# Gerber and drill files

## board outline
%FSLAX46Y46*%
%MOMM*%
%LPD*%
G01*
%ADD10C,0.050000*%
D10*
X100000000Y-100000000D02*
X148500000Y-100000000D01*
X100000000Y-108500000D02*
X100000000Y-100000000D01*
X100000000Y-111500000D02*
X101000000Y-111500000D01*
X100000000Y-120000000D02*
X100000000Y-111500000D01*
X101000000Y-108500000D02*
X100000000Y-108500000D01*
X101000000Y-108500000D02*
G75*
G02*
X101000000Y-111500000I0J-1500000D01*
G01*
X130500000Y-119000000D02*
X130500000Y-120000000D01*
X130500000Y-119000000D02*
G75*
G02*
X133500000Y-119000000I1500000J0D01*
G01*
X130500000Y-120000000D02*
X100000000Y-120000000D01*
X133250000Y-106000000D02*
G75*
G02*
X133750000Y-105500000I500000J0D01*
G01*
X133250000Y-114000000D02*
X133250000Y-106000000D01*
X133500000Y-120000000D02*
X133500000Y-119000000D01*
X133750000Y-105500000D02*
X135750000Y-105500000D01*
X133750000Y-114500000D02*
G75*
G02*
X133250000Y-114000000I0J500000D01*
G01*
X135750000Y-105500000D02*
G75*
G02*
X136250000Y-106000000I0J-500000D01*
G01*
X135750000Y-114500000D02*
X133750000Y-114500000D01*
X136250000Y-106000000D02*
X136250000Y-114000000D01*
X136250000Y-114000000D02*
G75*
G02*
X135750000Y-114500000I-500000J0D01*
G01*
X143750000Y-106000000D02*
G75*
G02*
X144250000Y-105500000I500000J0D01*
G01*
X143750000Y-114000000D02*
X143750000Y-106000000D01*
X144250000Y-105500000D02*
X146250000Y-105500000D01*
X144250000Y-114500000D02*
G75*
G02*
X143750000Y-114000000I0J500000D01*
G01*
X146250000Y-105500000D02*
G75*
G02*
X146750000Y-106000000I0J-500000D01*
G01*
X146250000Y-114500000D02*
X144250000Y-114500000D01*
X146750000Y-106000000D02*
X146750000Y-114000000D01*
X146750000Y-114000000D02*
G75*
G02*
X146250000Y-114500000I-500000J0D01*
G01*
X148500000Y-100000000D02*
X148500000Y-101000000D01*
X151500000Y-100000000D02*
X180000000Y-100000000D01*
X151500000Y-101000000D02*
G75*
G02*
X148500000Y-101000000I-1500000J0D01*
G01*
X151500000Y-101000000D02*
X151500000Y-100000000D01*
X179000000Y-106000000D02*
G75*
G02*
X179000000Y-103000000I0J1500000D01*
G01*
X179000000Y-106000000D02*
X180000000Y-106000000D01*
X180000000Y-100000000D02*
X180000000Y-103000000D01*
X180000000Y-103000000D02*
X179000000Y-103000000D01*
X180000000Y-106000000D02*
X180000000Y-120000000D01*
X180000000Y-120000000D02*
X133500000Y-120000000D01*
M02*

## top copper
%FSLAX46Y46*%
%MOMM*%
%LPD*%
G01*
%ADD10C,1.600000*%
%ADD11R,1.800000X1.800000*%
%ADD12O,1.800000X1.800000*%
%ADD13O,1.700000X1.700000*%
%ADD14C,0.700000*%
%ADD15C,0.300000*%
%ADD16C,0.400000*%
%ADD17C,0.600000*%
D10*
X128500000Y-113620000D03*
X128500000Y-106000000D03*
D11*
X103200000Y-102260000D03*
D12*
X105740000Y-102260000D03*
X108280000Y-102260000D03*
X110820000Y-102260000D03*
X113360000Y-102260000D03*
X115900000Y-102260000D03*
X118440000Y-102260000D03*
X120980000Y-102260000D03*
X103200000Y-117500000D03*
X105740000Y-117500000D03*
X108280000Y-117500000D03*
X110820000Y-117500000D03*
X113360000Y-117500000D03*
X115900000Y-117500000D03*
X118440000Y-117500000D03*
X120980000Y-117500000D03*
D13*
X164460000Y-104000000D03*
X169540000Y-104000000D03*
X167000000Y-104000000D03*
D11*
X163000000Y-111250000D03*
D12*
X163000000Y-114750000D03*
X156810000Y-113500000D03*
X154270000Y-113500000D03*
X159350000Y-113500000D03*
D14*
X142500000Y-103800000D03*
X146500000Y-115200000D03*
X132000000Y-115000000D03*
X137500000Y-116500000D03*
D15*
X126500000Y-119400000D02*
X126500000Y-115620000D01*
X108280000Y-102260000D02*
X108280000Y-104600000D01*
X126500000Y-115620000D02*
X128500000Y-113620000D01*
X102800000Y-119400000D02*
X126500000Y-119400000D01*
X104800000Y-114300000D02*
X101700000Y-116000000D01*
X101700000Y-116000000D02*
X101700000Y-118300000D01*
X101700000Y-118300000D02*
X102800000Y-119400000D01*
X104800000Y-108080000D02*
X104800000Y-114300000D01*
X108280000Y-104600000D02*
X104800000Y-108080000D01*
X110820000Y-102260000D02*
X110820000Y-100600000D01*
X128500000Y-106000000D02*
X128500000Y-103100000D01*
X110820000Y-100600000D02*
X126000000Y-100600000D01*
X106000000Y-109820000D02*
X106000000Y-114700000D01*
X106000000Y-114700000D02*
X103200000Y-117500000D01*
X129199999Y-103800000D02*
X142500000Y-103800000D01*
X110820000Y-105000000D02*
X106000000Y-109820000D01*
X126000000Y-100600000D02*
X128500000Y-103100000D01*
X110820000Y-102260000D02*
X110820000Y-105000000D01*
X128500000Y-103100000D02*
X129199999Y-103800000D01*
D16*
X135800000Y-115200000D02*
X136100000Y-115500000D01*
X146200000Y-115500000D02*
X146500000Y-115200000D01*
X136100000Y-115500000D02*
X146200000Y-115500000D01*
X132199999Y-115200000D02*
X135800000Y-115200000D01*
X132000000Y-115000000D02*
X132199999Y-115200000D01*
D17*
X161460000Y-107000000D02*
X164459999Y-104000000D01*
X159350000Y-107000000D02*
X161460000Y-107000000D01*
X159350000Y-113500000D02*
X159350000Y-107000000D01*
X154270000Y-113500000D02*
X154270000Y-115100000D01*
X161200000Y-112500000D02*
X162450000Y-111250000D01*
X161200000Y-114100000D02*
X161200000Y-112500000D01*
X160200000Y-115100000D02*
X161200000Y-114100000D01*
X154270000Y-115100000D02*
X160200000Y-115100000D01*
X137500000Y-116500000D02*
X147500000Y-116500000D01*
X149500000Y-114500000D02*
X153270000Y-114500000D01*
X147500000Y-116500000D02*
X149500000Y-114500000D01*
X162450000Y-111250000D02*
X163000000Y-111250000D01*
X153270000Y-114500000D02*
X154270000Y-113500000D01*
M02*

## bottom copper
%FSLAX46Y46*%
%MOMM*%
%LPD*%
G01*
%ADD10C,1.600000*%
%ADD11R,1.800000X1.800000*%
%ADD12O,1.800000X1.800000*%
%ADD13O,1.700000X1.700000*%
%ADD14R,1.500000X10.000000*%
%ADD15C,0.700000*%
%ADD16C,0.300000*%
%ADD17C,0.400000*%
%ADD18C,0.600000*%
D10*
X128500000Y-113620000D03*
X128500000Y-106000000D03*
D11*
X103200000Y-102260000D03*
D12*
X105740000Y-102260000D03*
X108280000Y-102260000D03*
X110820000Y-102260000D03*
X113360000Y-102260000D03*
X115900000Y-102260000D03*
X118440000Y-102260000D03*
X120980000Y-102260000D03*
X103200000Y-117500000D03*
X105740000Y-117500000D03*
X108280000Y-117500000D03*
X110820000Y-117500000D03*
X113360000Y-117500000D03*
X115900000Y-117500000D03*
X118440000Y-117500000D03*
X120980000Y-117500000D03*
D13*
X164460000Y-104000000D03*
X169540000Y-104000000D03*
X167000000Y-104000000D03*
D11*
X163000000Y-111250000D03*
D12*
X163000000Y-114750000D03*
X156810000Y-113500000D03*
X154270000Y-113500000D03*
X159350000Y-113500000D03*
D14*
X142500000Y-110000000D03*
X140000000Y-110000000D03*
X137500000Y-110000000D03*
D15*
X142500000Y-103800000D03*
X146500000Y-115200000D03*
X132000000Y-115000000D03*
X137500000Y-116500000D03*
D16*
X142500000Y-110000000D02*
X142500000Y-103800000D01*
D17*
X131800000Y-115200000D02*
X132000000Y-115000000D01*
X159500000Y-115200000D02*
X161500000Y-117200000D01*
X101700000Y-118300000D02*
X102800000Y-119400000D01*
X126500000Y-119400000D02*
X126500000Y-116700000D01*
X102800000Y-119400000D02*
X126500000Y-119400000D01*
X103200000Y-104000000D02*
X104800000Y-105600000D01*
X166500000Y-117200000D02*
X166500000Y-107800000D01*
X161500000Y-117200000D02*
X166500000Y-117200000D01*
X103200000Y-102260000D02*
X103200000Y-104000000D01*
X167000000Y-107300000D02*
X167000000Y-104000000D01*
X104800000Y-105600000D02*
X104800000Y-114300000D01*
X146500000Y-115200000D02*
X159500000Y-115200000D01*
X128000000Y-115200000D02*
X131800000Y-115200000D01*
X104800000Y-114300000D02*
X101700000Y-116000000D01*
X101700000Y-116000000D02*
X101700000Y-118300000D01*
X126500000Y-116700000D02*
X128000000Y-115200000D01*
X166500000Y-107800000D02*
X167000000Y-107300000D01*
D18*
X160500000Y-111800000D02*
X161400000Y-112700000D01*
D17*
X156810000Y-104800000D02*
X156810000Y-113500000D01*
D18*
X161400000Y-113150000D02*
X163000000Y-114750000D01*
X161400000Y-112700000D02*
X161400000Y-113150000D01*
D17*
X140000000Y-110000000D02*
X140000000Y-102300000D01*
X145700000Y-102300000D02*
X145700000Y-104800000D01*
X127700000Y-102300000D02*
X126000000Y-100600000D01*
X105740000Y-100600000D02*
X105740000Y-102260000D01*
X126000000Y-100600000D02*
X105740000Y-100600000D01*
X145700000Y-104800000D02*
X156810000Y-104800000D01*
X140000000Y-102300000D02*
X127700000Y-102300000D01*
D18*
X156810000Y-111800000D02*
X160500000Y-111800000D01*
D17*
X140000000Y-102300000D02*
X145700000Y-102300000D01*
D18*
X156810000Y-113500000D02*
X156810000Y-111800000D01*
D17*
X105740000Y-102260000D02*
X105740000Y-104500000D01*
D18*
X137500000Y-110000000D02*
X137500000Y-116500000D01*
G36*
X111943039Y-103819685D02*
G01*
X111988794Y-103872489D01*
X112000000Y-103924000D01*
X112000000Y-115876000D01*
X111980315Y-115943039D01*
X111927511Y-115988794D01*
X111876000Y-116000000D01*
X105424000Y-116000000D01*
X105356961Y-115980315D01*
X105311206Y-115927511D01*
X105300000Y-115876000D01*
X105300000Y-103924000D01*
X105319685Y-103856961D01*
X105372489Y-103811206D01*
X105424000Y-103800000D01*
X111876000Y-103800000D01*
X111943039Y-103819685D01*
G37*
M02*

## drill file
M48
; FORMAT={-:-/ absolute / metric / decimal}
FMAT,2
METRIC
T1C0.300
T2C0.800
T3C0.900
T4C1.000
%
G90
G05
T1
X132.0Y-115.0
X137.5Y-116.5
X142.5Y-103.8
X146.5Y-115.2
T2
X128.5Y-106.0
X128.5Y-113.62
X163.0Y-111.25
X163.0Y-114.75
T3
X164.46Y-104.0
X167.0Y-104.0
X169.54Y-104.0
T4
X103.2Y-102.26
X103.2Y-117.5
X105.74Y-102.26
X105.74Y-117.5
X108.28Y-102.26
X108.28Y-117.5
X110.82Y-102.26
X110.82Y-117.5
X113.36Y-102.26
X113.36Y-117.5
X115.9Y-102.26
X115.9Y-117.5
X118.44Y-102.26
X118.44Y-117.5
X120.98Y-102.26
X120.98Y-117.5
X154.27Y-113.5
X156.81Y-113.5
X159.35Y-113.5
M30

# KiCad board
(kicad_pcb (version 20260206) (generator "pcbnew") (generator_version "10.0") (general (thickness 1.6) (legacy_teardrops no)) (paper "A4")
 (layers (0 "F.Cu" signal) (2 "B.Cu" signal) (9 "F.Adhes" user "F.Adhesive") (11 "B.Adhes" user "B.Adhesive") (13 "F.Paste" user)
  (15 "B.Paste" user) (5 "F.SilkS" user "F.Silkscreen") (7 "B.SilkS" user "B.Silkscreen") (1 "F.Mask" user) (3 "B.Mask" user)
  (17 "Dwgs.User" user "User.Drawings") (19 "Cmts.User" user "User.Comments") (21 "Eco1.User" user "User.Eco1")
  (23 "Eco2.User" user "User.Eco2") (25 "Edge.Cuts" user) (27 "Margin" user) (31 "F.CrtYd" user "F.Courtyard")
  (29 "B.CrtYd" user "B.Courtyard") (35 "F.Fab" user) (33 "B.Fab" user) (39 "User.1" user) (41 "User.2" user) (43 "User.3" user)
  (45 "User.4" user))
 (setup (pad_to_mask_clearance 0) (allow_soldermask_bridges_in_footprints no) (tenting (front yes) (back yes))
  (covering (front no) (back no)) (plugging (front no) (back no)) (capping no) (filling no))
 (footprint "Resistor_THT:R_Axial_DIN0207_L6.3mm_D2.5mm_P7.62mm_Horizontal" (layer "F.Cu") (at 128.5 113.62 90)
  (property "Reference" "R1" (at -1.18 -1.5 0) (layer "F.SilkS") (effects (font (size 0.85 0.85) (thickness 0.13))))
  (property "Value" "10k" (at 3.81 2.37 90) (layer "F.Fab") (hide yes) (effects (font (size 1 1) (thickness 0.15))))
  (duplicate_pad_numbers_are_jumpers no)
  (pad "1" thru_hole circle (at 0 0 90) (size 1.6 1.6) (drill 0.8) (layers "*.Cu" "*.Mask") (remove_unused_layers no) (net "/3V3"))
  (pad "2" thru_hole circle (at 7.62 0 90) (size 1.6 1.6) (drill 0.8) (layers "*.Cu" "*.Mask") (remove_unused_layers no) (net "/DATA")))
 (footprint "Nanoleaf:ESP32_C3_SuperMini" (layer "F.Cu") (at 103.2 117.5 90)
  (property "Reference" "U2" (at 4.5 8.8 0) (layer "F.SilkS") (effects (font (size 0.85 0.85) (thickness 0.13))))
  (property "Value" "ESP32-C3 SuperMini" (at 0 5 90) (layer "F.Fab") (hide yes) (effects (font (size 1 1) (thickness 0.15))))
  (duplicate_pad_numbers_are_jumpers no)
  (pad "1" thru_hole rect (at 15.24 0 90) (size 1.8 1.8) (drill 1) (layers "*.Cu" "*.Mask") (remove_unused_layers no) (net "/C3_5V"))
  (pad "2" thru_hole oval (at 15.24 2.54 90) (size 1.8 1.8) (drill 1) (layers "*.Cu" "*.Mask") (remove_unused_layers no) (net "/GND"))
  (pad "3" thru_hole oval (at 15.24 5.08 90) (size 1.8 1.8) (drill 1) (layers "*.Cu" "*.Mask") (remove_unused_layers no) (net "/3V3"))
  (pad "4" thru_hole oval (at 15.24 7.62 90) (size 1.8 1.8) (drill 1) (layers "*.Cu" "*.Mask") (remove_unused_layers no) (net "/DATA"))
  (pad "5" thru_hole oval (at 15.24 10.16 90) (size 1.8 1.8) (drill 1) (layers "*.Cu" "*.Mask") (remove_unused_layers no)
   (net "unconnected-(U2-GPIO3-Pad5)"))
  (pad "6" thru_hole oval (at 15.24 12.7 90) (size 1.8 1.8) (drill 1) (layers "*.Cu" "*.Mask") (remove_unused_layers no)
   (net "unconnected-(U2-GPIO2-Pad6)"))
  (pad "7" thru_hole oval (at 15.24 15.24 90) (size 1.8 1.8) (drill 1) (layers "*.Cu" "*.Mask") (remove_unused_layers no)
   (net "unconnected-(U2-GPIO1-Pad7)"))
  (pad "8" thru_hole oval (at 15.24 17.78 90) (size 1.8 1.8) (drill 1) (layers "*.Cu" "*.Mask") (remove_unused_layers no)
   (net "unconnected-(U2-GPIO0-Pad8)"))
  (pad "9" thru_hole oval (at 0 0 90) (size 1.8 1.8) (drill 1) (layers "*.Cu" "*.Mask") (remove_unused_layers no) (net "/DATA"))
  (pad "10" thru_hole oval (at 0 2.54 90) (size 1.8 1.8) (drill 1) (layers "*.Cu" "*.Mask") (remove_unused_layers no)
   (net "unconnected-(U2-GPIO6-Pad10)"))
  (pad "11" thru_hole oval (at 0 5.08 90) (size 1.8 1.8) (drill 1) (layers "*.Cu" "*.Mask") (remove_unused_layers no)
   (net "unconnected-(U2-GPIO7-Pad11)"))
  (pad "12" thru_hole oval (at 0 7.62 90) (size 1.8 1.8) (drill 1) (layers "*.Cu" "*.Mask") (remove_unused_layers no)
   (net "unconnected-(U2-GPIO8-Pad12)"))
  (pad "13" thru_hole oval (at 0 10.16 90) (size 1.8 1.8) (drill 1) (layers "*.Cu" "*.Mask") (remove_unused_layers no)
   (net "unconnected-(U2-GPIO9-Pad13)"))
  (pad "14" thru_hole oval (at 0 12.7 90) (size 1.8 1.8) (drill 1) (layers "*.Cu" "*.Mask") (remove_unused_layers no)
   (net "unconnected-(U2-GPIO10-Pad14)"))
  (pad "15" thru_hole oval (at 0 15.24 90) (size 1.8 1.8) (drill 1) (layers "*.Cu" "*.Mask") (remove_unused_layers no)
   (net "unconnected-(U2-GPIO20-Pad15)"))
  (pad "16" thru_hole oval (at 0 17.78 90) (size 1.8 1.8) (drill 1) (layers "*.Cu" "*.Mask") (remove_unused_layers no)
   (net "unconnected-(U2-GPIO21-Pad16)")))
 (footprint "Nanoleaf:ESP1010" (layer "F.Cu") (at 167 104)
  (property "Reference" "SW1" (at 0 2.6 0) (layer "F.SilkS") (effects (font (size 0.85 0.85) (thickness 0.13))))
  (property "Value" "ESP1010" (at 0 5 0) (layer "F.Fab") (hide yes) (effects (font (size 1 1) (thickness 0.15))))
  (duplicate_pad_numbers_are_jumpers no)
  (pad "1" thru_hole oval (at -2.54 0) (size 1.7 1.7) (drill 0.9) (layers "*.Cu" "*.Mask") (remove_unused_layers no) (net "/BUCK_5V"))
  (pad "2" thru_hole oval (at 2.54 0) (size 1.7 1.7) (drill 0.9) (layers "*.Cu" "*.Mask") (remove_unused_layers no)
   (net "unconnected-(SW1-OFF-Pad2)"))
  (pad "C" thru_hole oval (at 0 0) (size 1.7 1.7) (drill 0.9) (layers "*.Cu" "*.Mask") (remove_unused_layers no) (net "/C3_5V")))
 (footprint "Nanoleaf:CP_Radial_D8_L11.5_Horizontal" (layer "F.Cu") (at 163 111.25)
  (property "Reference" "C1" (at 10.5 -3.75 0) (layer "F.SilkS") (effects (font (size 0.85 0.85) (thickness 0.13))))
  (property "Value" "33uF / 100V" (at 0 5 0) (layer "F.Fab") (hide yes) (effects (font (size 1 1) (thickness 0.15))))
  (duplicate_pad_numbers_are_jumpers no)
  (pad "1" thru_hole rect (at 0 0) (size 1.8 1.8) (drill 0.8) (layers "*.Cu" "*.Mask") (remove_unused_layers no) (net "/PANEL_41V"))
  (pad "2" thru_hole oval (at 0 3.5) (size 1.8 1.8) (drill 0.8) (layers "*.Cu" "*.Mask") (remove_unused_layers no) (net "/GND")))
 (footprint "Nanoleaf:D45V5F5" (layer "F.Cu") (at 154.27 113.5)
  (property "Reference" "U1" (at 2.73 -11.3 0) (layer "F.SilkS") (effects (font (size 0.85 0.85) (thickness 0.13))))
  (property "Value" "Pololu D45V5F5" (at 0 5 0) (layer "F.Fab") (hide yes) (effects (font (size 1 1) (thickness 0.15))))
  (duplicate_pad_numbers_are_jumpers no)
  (pad "GND" thru_hole oval (at 2.54 0) (size 1.8 1.8) (drill 1) (layers "*.Cu" "*.Mask") (remove_unused_layers no) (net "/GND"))
  (pad "VIN" thru_hole oval (at 0 0) (size 1.8 1.8) (drill 1) (layers "*.Cu" "*.Mask") (remove_unused_layers no) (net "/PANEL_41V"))
  (pad "VOUT" thru_hole oval (at 5.08 0) (size 1.8 1.8) (drill 1) (layers "*.Cu" "*.Mask") (remove_unused_layers no) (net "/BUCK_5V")))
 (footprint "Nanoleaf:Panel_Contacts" (layer "B.Cu") (at 140 110 180)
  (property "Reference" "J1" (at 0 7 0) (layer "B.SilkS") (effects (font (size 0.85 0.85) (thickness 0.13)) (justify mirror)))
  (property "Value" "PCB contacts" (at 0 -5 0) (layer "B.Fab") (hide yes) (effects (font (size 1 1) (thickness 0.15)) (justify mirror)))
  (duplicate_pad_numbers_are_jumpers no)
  (pad "1" smd rect (at -2.5 0 180) (size 1.5 10) (layers "B.Cu" "B.Mask") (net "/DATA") (solder_mask_margin 0) (clearance 0.4))
  (pad "2" smd rect (at 0 0 180) (size 1.5 10) (layers "B.Cu" "B.Mask") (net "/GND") (solder_mask_margin 0) (clearance 0.4))
  (pad "3" smd rect (at 2.5 0 180) (size 1.5 10) (layers "B.Cu" "B.Mask") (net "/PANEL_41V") (solder_mask_margin 0) (clearance 0.4)))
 (gr_line (start 100 100) (end 148.5 100) (stroke (width 0.05) (type default)) (layer "Edge.Cuts"))
 (gr_line (start 100 108.5) (end 100 100) (stroke (width 0.05) (type default)) (layer "Edge.Cuts"))
 (gr_line (start 100 111.5) (end 101 111.5) (stroke (width 0.05) (type default)) (layer "Edge.Cuts"))
 (gr_line (start 100 120) (end 100 111.5) (stroke (width 0.05) (type default)) (layer "Edge.Cuts"))
 (gr_line (start 101 108.5) (end 100 108.5) (stroke (width 0.05) (type default)) (layer "Edge.Cuts"))
 (gr_arc (start 101 108.5) (mid 102.5 110) (end 101 111.5) (stroke (width 0.05) (type default)) (layer "Edge.Cuts"))
 (gr_line (start 130.5 119) (end 130.5 120) (stroke (width 0.05) (type default)) (layer "Edge.Cuts"))
 (gr_arc (start 130.5 119) (mid 132 117.5) (end 133.5 119) (stroke (width 0.05) (type default)) (layer "Edge.Cuts"))
 (gr_line (start 130.5 120) (end 100 120) (stroke (width 0.05) (type default)) (layer "Edge.Cuts"))
 (gr_arc (start 133.25 106) (mid 133.396446 105.646446) (end 133.75 105.5) (stroke (width 0.05) (type default)) (layer "Edge.Cuts"))
 (gr_line (start 133.25 114) (end 133.25 106) (stroke (width 0.05) (type default)) (layer "Edge.Cuts"))
 (gr_line (start 133.5 120) (end 133.5 119) (stroke (width 0.05) (type default)) (layer "Edge.Cuts"))
 (gr_line (start 133.75 105.5) (end 135.75 105.5) (stroke (width 0.05) (type default)) (layer "Edge.Cuts"))
 (gr_arc (start 133.75 114.5) (mid 133.396446 114.353553) (end 133.25 114) (stroke (width 0.05) (type default)) (layer "Edge.Cuts"))
 (gr_arc (start 135.75 105.5) (mid 136.103553 105.646446) (end 136.25 106) (stroke (width 0.05) (type default)) (layer "Edge.Cuts"))
 (gr_line (start 135.75 114.5) (end 133.75 114.5) (stroke (width 0.05) (type default)) (layer "Edge.Cuts"))
 (gr_line (start 136.25 106) (end 136.25 114) (stroke (width 0.05) (type default)) (layer "Edge.Cuts"))
 (gr_arc (start 136.25 114) (mid 136.103553 114.353553) (end 135.75 114.5) (stroke (width 0.05) (type default)) (layer "Edge.Cuts"))
 (gr_arc (start 143.75 106) (mid 143.896446 105.646446) (end 144.25 105.5) (stroke (width 0.05) (type default)) (layer "Edge.Cuts"))
 (gr_line (start 143.75 114) (end 143.75 106) (stroke (width 0.05) (type default)) (layer "Edge.Cuts"))
 (gr_line (start 144.25 105.5) (end 146.25 105.5) (stroke (width 0.05) (type default)) (layer "Edge.Cuts"))
 (gr_arc (start 144.25 114.5) (mid 143.896446 114.353553) (end 143.75 114) (stroke (width 0.05) (type default)) (layer "Edge.Cuts"))
 (gr_arc (start 146.25 105.5) (mid 146.603553 105.646446) (end 146.75 106) (stroke (width 0.05) (type default)) (layer "Edge.Cuts"))
 (gr_line (start 146.25 114.5) (end 144.25 114.5) (stroke (width 0.05) (type default)) (layer "Edge.Cuts"))
 (gr_line (start 146.75 106) (end 146.75 114) (stroke (width 0.05) (type default)) (layer "Edge.Cuts"))
 (gr_arc (start 146.75 114) (mid 146.603553 114.353553) (end 146.25 114.5) (stroke (width 0.05) (type default)) (layer "Edge.Cuts"))
 (gr_line (start 148.5 100) (end 148.5 101) (stroke (width 0.05) (type default)) (layer "Edge.Cuts"))
 (gr_line (start 151.5 100) (end 180 100) (stroke (width 0.05) (type default)) (layer "Edge.Cuts"))
 (gr_arc (start 151.5 101) (mid 150 102.5) (end 148.5 101) (stroke (width 0.05) (type default)) (layer "Edge.Cuts"))
 (gr_line (start 151.5 101) (end 151.5 100) (stroke (width 0.05) (type default)) (layer "Edge.Cuts"))
 (gr_arc (start 179 106) (mid 177.5 104.5) (end 179 103) (stroke (width 0.05) (type default)) (layer "Edge.Cuts"))
 (gr_line (start 179 106) (end 180 106) (stroke (width 0.05) (type default)) (layer "Edge.Cuts"))
 (gr_line (start 180 100) (end 180 103) (stroke (width 0.05) (type default)) (layer "Edge.Cuts"))
 (gr_line (start 180 103) (end 179 103) (stroke (width 0.05) (type default)) (layer "Edge.Cuts"))
 (gr_line (start 180 106) (end 180 120) (stroke (width 0.05) (type default)) (layer "Edge.Cuts"))
 (gr_line (start 180 120) (end 133.5 120) (stroke (width 0.05) (type default)) (layer "Edge.Cuts"))
 (segment (start 126.5 119.4) (end 126.5 115.62) (width 0.3) (layer "F.Cu") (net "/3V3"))
 (segment (start 108.28 102.26) (end 108.28 104.6) (width 0.3) (layer "F.Cu") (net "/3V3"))
 (segment (start 126.5 115.62) (end 128.5 113.62) (width 0.3) (layer "F.Cu") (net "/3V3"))
 (segment (start 102.8 119.4) (end 126.5 119.4) (width 0.3) (layer "F.Cu") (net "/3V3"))
 (segment (start 104.8 114.3) (end 101.7 116) (width 0.3) (layer "F.Cu") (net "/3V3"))
 (segment (start 101.7 116) (end 101.7 118.3) (width 0.3) (layer "F.Cu") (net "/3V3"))
 (segment (start 101.7 118.3) (end 102.8 119.4) (width 0.3) (layer "F.Cu") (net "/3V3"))
 (segment (start 104.8 108.08) (end 104.8 114.3) (width 0.3) (layer "F.Cu") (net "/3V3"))
 (segment (start 108.28 104.6) (end 104.8 108.08) (width 0.3) (layer "F.Cu") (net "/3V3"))
 (segment (start 110.82 102.26) (end 110.82 100.6) (width 0.3) (layer "F.Cu") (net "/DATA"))
 (segment (start 128.5 106) (end 128.5 103.1) (width 0.3) (layer "F.Cu") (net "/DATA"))
 (segment (start 110.82 100.6) (end 126 100.6) (width 0.3) (layer "F.Cu") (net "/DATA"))
 (segment (start 106 109.82) (end 106 114.7) (width 0.3) (layer "F.Cu") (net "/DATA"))
 (segment (start 106 114.7) (end 103.2 117.5) (width 0.3) (layer "F.Cu") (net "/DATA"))
 (segment (start 129.199999 103.8) (end 142.5 103.8) (width 0.3) (layer "F.Cu") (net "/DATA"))
 (segment (start 110.82 105) (end 106 109.82) (width 0.3) (layer "F.Cu") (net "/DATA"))
 (segment (start 126 100.6) (end 128.5 103.1) (width 0.3) (layer "F.Cu") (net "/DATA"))
 (segment (start 110.82 102.26) (end 110.82 105) (width 0.3) (layer "F.Cu") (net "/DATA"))
 (segment (start 128.5 103.1) (end 129.199999 103.8) (width 0.3) (layer "F.Cu") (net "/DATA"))
 (via (at 142.5 103.8) (size 0.7) (drill 0.3) (layers "F.Cu" "B.Cu") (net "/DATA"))
 (segment (start 142.5 110) (end 142.5 103.8) (width 0.3) (layer "B.Cu") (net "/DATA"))
 (segment (start 135.8 115.2) (end 136.1 115.5) (width 0.4) (layer "F.Cu") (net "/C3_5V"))
 (segment (start 146.2 115.5) (end 146.5 115.2) (width 0.4) (layer "F.Cu") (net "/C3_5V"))
 (segment (start 136.1 115.5) (end 146.2 115.5) (width 0.4) (layer "F.Cu") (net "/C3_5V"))
 (segment (start 132.199999 115.2) (end 135.8 115.2) (width 0.4) (layer "F.Cu") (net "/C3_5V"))
 (segment (start 132 115) (end 132.199999 115.2) (width 0.4) (layer "F.Cu") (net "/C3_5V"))
 (via (at 146.5 115.2) (size 0.7) (drill 0.3) (layers "F.Cu" "B.Cu") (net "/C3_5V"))
 (via (at 132 115) (size 0.7) (drill 0.3) (layers "F.Cu" "B.Cu") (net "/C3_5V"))
 (segment (start 131.8 115.2) (end 132 115) (width 0.4) (layer "B.Cu") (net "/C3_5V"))
 (segment (start 159.5 115.2) (end 161.5 117.2) (width 0.4) (layer "B.Cu") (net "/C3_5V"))
 (segment (start 101.7 118.3) (end 102.8 119.4) (width 0.4) (layer "B.Cu") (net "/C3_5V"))
 (segment (start 126.5 119.4) (end 126.5 116.7) (width 0.4) (layer "B.Cu") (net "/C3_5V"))
 (segment (start 102.8 119.4) (end 126.5 119.4) (width 0.4) (layer "B.Cu") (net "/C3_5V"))
 (segment (start 103.2 104) (end 104.8 105.6) (width 0.4) (layer "B.Cu") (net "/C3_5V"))
 (segment (start 166.5 117.2) (end 166.5 107.8) (width 0.4) (layer "B.Cu") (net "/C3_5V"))
 (segment (start 161.5 117.2) (end 166.5 117.2) (width 0.4) (layer "B.Cu") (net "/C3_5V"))
 (segment (start 103.2 102.26) (end 103.2 104) (width 0.4) (layer "B.Cu") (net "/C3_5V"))
 (segment (start 167 107.3) (end 167 104) (width 0.4) (layer "B.Cu") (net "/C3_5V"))
 (segment (start 104.8 105.6) (end 104.8 114.3) (width 0.4) (layer "B.Cu") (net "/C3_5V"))
 (segment (start 146.5 115.2) (end 159.5 115.2) (width 0.4) (layer "B.Cu") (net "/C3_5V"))
 (segment (start 128 115.2) (end 131.8 115.2) (width 0.4) (layer "B.Cu") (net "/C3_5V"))
 (segment (start 104.8 114.3) (end 101.7 116) (width 0.4) (layer "B.Cu") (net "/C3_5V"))
 (segment (start 101.7 116) (end 101.7 118.3) (width 0.4) (layer "B.Cu") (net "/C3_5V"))
 (segment (start 126.5 116.7) (end 128 115.2) (width 0.4) (layer "B.Cu") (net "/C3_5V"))
 (segment (start 166.5 107.8) (end 167 107.3) (width 0.4) (layer "B.Cu") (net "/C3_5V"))
 (segment (start 160.5 111.8) (end 161.4 112.7) (width 0.6) (layer "B.Cu") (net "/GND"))
 (segment (start 156.81 104.8) (end 156.81 113.5) (width 0.4) (layer "B.Cu") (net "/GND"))
 (segment (start 161.4 113.15) (end 163 114.75) (width 0.6) (layer "B.Cu") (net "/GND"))
 (segment (start 161.4 112.7) (end 161.4 113.15) (width 0.6) (layer "B.Cu") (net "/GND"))
 (segment (start 140 110) (end 140 102.3) (width 0.4) (layer "B.Cu") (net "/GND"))
 (segment (start 145.7 102.3) (end 145.7 104.8) (width 0.4) (layer "B.Cu") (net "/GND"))
 (segment (start 127.7 102.3) (end 126 100.6) (width 0.4) (layer "B.Cu") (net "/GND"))
 (segment (start 105.74 100.6) (end 105.74 102.26) (width 0.4) (layer "B.Cu") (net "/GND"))
 (segment (start 126 100.6) (end 105.74 100.6) (width 0.4) (layer "B.Cu") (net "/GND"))
 (segment (start 145.7 104.8) (end 156.81 104.8) (width 0.4) (layer "B.Cu") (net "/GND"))
 (segment (start 140 102.3) (end 127.7 102.3) (width 0.4) (layer "B.Cu") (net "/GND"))
 (segment (start 156.81 111.8) (end 160.5 111.8) (width 0.6) (layer "B.Cu") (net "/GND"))
 (segment (start 140 102.3) (end 145.7 102.3) (width 0.4) (layer "B.Cu") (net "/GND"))
 (segment (start 156.81 113.5) (end 156.81 111.8) (width 0.6) (layer "B.Cu") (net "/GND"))
 (segment (start 105.74 102.26) (end 105.74 104.5) (width 0.4) (layer "B.Cu") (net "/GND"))
 (segment (start 161.46 107) (end 164.459999 104) (width 0.6) (layer "F.Cu") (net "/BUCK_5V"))
 (segment (start 159.35 107) (end 161.46 107) (width 0.6) (layer "F.Cu") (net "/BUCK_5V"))
 (segment (start 159.35 113.5) (end 159.35 107) (width 0.6) (layer "F.Cu") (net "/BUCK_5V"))
 (segment (start 154.27 113.5) (end 154.27 115.1) (width 0.6) (layer "F.Cu") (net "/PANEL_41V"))
 (segment (start 161.2 112.5) (end 162.45 111.25) (width 0.6) (layer "F.Cu") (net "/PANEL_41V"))
 (segment (start 161.2 114.1) (end 161.2 112.5) (width 0.6) (layer "F.Cu") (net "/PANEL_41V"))
 (segment (start 160.2 115.1) (end 161.2 114.1) (width 0.6) (layer "F.Cu") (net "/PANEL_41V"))
 (segment (start 154.27 115.1) (end 160.2 115.1) (width 0.6) (layer "F.Cu") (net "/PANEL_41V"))
 (segment (start 137.5 116.5) (end 147.5 116.5) (width 0.6) (layer "F.Cu") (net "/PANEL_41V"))
 (segment (start 149.5 114.5) (end 153.27 114.5) (width 0.6) (layer "F.Cu") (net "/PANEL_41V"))
 (segment (start 147.5 116.5) (end 149.5 114.5) (width 0.6) (layer "F.Cu") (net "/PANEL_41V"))
 (segment (start 162.45 111.25) (end 163 111.25) (width 0.6) (layer "F.Cu") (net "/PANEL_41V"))
 (segment (start 153.27 114.5) (end 154.27 113.5) (width 0.6) (layer "F.Cu") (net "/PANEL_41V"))
 (via (at 137.5 116.5) (size 0.7) (drill 0.3) (layers "F.Cu" "B.Cu") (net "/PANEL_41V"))
 (segment (start 137.5 110) (end 137.5 116.5) (width 0.6) (layer "B.Cu") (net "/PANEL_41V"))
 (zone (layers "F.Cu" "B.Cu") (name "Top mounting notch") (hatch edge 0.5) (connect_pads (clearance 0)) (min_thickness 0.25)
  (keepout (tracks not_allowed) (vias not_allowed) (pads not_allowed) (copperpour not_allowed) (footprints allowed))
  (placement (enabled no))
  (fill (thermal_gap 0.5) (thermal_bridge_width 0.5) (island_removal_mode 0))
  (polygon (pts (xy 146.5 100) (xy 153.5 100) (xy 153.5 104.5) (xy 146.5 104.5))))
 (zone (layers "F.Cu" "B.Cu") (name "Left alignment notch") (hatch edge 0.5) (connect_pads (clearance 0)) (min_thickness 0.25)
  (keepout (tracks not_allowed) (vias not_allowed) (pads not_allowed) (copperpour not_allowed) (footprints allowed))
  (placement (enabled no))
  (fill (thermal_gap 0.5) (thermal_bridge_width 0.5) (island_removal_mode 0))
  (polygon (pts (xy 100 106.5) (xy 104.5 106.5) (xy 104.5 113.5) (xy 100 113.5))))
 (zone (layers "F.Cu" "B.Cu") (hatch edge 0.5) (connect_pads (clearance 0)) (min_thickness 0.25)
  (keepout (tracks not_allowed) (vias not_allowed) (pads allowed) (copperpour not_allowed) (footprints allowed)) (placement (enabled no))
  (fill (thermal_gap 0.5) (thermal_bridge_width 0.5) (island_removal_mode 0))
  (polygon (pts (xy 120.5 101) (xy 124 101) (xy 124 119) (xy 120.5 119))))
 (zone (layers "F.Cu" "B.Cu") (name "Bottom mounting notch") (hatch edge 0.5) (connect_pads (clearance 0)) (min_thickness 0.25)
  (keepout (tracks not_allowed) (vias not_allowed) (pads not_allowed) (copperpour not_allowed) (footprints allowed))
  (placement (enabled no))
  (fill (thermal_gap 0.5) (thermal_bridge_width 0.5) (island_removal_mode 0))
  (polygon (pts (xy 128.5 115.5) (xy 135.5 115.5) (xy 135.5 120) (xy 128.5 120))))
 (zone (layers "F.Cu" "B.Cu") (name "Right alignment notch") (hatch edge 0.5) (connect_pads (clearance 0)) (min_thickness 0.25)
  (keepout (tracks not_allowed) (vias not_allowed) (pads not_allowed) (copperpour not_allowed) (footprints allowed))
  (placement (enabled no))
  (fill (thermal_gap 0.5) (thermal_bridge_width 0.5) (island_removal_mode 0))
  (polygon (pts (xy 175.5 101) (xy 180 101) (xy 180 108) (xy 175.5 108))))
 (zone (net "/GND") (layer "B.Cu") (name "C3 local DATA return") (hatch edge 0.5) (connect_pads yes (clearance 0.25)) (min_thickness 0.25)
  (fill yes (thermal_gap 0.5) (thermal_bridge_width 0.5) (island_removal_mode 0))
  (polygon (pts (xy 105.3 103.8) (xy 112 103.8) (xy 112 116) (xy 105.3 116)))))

